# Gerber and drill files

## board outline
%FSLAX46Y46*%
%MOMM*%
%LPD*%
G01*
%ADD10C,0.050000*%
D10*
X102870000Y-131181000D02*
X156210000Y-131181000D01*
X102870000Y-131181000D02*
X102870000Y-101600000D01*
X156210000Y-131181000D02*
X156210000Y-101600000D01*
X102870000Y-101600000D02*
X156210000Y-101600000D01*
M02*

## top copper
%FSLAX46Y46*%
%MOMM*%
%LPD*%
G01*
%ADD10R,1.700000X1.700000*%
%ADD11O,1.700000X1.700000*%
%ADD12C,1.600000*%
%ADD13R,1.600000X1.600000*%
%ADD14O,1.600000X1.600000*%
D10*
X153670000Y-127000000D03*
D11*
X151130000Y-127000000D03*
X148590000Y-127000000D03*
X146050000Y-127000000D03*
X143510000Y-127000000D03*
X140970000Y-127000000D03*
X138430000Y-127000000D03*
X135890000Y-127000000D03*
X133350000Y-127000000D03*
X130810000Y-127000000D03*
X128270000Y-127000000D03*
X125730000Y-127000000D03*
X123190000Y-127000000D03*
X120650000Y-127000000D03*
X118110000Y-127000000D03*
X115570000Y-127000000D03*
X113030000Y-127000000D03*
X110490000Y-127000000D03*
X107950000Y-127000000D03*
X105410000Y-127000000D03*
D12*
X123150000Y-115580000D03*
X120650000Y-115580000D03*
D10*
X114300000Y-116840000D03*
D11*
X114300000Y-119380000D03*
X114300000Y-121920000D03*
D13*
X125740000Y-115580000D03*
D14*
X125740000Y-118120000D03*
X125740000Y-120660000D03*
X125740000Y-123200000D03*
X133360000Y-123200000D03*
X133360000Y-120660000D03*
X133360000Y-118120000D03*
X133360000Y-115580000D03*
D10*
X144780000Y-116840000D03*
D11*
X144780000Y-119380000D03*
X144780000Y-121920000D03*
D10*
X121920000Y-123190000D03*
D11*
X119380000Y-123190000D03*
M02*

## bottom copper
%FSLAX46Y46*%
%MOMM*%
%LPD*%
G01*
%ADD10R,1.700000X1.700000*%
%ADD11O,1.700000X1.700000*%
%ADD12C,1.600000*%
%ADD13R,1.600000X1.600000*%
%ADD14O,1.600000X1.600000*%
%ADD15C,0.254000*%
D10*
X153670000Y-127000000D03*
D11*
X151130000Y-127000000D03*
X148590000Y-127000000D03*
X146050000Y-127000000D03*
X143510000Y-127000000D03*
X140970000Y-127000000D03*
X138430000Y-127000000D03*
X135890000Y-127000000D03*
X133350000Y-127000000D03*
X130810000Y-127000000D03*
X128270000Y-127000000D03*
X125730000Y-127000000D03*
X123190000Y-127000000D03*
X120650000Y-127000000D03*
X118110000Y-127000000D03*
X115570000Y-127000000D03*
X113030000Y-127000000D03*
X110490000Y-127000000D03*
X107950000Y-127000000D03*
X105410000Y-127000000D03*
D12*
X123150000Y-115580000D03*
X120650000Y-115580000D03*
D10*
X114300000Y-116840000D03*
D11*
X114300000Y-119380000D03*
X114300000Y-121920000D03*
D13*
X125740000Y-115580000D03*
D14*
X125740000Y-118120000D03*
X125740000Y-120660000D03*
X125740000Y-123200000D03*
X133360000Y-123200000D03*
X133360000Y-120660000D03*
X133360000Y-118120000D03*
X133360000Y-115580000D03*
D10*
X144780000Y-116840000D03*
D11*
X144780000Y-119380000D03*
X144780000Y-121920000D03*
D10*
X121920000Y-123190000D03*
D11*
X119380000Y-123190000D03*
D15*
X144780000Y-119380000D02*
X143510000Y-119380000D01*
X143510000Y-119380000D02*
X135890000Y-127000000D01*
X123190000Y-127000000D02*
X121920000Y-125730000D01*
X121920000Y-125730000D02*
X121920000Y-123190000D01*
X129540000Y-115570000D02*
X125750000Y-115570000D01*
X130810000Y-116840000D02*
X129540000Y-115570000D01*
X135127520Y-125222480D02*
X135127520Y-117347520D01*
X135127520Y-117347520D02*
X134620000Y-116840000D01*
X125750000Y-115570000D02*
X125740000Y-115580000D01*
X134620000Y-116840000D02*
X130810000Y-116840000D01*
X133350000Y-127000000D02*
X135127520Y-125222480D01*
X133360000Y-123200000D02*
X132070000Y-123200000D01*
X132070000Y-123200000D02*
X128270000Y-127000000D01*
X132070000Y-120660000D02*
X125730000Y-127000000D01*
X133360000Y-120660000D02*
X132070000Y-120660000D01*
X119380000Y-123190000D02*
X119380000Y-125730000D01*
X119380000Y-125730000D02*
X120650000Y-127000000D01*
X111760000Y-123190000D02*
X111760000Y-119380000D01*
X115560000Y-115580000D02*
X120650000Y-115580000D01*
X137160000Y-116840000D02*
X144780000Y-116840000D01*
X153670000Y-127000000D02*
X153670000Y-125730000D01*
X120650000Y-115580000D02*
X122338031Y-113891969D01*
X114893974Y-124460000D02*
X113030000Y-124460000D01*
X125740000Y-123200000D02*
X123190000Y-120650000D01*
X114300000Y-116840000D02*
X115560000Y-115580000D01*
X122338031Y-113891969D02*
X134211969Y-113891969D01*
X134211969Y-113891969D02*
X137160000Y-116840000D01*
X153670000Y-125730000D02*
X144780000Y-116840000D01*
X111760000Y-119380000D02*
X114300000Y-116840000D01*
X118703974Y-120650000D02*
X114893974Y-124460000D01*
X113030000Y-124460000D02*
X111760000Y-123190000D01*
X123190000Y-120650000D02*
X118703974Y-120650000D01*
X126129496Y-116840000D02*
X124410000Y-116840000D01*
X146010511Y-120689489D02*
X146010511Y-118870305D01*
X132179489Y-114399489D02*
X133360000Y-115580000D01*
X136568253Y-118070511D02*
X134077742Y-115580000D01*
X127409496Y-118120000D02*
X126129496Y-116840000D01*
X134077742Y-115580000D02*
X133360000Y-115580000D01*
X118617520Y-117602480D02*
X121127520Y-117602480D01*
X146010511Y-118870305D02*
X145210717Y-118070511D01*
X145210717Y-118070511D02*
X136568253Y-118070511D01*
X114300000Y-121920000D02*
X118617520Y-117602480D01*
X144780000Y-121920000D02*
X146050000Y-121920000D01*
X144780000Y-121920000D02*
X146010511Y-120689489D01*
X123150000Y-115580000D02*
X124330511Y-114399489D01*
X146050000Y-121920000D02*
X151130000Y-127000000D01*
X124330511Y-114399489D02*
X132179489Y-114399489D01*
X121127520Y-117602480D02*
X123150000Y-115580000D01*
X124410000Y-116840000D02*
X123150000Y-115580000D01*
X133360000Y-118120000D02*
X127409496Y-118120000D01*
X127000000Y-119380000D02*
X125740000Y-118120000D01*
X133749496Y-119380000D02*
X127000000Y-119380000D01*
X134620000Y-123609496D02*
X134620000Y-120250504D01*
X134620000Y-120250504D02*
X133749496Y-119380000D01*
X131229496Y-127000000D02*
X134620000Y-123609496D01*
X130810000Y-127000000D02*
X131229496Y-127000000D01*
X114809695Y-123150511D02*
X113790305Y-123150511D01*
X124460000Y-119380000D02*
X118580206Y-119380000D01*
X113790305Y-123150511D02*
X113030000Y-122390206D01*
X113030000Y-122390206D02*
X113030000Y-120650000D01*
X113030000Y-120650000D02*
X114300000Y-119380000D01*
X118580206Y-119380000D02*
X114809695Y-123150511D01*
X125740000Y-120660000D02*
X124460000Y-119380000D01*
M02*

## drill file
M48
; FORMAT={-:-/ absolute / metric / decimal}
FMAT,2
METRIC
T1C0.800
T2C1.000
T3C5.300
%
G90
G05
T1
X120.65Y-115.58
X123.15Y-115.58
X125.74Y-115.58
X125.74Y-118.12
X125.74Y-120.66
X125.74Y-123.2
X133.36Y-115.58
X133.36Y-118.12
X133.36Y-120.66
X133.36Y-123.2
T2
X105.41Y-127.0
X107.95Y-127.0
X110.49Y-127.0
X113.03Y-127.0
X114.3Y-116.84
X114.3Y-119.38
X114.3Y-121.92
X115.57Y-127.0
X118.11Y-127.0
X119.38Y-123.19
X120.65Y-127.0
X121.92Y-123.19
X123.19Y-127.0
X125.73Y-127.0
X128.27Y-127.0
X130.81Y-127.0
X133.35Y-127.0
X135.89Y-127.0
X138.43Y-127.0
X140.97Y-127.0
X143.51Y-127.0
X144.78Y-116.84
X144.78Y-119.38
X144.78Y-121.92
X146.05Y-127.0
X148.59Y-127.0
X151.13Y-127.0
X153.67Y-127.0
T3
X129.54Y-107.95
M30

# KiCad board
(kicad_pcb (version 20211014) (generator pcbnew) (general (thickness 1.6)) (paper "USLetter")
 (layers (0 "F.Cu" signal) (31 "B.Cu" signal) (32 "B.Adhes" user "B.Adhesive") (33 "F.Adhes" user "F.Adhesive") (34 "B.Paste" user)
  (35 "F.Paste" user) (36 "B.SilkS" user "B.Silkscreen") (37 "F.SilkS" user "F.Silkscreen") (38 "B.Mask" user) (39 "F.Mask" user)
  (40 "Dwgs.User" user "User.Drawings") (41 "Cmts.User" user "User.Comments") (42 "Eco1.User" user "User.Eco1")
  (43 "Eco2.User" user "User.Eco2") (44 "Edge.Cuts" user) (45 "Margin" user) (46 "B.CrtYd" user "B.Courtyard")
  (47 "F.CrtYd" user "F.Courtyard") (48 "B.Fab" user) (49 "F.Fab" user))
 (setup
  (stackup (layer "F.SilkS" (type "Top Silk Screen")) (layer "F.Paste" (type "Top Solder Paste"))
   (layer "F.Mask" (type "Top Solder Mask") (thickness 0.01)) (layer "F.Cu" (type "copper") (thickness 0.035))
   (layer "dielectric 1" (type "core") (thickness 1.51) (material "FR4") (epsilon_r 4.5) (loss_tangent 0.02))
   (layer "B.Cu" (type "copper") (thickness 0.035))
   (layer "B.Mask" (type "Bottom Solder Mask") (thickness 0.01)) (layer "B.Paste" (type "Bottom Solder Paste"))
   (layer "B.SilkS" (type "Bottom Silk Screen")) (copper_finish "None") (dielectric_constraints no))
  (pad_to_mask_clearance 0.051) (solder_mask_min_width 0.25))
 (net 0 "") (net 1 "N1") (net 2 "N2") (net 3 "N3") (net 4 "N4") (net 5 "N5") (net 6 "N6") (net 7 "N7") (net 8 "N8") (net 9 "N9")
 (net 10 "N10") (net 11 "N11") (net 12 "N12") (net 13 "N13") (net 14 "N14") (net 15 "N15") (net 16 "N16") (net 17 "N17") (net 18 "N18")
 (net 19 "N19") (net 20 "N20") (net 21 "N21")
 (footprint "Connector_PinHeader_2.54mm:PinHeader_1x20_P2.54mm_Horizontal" (layer "F.Cu") (at 153.67 127 -90)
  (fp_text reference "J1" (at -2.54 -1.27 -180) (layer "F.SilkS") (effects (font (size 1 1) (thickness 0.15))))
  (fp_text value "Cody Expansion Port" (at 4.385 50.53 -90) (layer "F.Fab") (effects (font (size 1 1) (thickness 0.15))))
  (pad "1" thru_hole rect (at 0 0 270) (size 1.7 1.7) (drill 1) (layers *.Cu *.Mask) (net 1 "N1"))
  (pad "2" thru_hole oval (at 0 2.54 270) (size 1.7 1.7) (drill 1) (layers *.Cu *.Mask) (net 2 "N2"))
  (pad "3" thru_hole oval (at 0 5.08 270) (size 1.7 1.7) (drill 1) (layers *.Cu *.Mask) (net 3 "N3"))
  (pad "4" thru_hole oval (at 0 7.62 270) (size 1.7 1.7) (drill 1) (layers *.Cu *.Mask) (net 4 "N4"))
  (pad "5" thru_hole oval (at 0 10.16 270) (size 1.7 1.7) (drill 1) (layers *.Cu *.Mask) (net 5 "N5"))
  (pad "6" thru_hole oval (at 0 12.7 270) (size 1.7 1.7) (drill 1) (layers *.Cu *.Mask) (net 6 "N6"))
  (pad "7" thru_hole oval (at 0 15.24 270) (size 1.7 1.7) (drill 1) (layers *.Cu *.Mask) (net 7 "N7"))
  (pad "8" thru_hole oval (at 0 17.78 270) (size 1.7 1.7) (drill 1) (layers *.Cu *.Mask) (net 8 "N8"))
  (pad "9" thru_hole oval (at 0 20.32 270) (size 1.7 1.7) (drill 1) (layers *.Cu *.Mask) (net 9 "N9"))
  (pad "10" thru_hole oval (at 0 22.86 270) (size 1.7 1.7) (drill 1) (layers *.Cu *.Mask) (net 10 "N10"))
  (pad "11" thru_hole oval (at 0 25.4 270) (size 1.7 1.7) (drill 1) (layers *.Cu *.Mask) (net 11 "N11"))
  (pad "12" thru_hole oval (at 0 27.94 270) (size 1.7 1.7) (drill 1) (layers *.Cu *.Mask) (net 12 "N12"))
  (pad "13" thru_hole oval (at 0 30.48 270) (size 1.7 1.7) (drill 1) (layers *.Cu *.Mask) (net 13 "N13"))
  (pad "14" thru_hole oval (at 0 33.02 270) (size 1.7 1.7) (drill 1) (layers *.Cu *.Mask) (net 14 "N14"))
  (pad "15" thru_hole oval (at 0 35.56 270) (size 1.7 1.7) (drill 1) (layers *.Cu *.Mask) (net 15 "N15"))
  (pad "16" thru_hole oval (at 0 38.1 270) (size 1.7 1.7) (drill 1) (layers *.Cu *.Mask) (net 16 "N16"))
  (pad "17" thru_hole oval (at 0 40.64 270) (size 1.7 1.7) (drill 1) (layers *.Cu *.Mask) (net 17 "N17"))
  (pad "18" thru_hole oval (at 0 43.18 270) (size 1.7 1.7) (drill 1) (layers *.Cu *.Mask) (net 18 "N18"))
  (pad "19" thru_hole oval (at 0 45.72 270) (size 1.7 1.7) (drill 1) (layers *.Cu *.Mask) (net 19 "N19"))
  (pad "20" thru_hole oval (at 0 48.26 270) (size 1.7 1.7) (drill 1) (layers *.Cu *.Mask) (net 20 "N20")))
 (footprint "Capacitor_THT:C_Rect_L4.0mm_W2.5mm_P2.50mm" (layer "F.Cu") (at 123.15 115.58 180)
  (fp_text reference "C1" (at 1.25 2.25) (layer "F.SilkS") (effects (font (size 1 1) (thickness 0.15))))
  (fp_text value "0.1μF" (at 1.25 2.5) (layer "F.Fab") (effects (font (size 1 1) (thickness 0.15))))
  (pad "1" thru_hole circle (at 0 0 180) (size 1.6 1.6) (drill 0.8) (layers *.Cu *.Mask) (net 2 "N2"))
  (pad "2" thru_hole circle (at 2.5 0 180) (size 1.6 1.6) (drill 0.8) (layers *.Cu *.Mask) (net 1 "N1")))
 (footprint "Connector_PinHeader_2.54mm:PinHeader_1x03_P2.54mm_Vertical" (layer "F.Cu") (at 114.3 116.84)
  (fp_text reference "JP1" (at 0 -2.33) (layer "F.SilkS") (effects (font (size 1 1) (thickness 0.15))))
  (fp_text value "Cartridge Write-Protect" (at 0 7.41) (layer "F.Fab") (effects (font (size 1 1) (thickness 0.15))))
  (pad "1" thru_hole rect (at 0 0) (size 1.7 1.7) (drill 1) (layers *.Cu *.Mask) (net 1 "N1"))
  (pad "2" thru_hole oval (at 0 2.54) (size 1.7 1.7) (drill 1) (layers *.Cu *.Mask) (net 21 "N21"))
  (pad "3" thru_hole oval (at 0 5.08) (size 1.7 1.7) (drill 1) (layers *.Cu *.Mask) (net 2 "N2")))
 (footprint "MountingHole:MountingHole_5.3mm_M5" (layer "F.Cu") (at 129.54 107.95)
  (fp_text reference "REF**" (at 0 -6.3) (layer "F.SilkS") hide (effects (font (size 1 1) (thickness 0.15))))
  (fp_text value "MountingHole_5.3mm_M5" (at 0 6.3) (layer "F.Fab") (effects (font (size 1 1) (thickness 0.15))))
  (pad "" np_thru_hole circle (at 0 0) (size 5.3 5.3) (drill 5.3) (layers *.Cu *.Mask)))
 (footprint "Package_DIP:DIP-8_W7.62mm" (layer "F.Cu") (at 125.74 115.58)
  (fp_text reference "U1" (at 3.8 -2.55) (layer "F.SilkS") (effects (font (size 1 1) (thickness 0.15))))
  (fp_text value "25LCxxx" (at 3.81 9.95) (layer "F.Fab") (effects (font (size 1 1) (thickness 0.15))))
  (pad "1" thru_hole rect (at 0 0) (size 1.6 1.6) (drill 0.8) (layers *.Cu *.Mask) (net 9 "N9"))
  (pad "2" thru_hole oval (at 0 2.54) (size 1.6 1.6) (drill 0.8) (layers *.Cu *.Mask) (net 10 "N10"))
  (pad "3" thru_hole oval (at 0 5.08) (size 1.6 1.6) (drill 0.8) (layers *.Cu *.Mask) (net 21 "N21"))
  (pad "4" thru_hole oval (at 0 7.62) (size 1.6 1.6) (drill 0.8) (layers *.Cu *.Mask) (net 1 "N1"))
  (pad "5" thru_hole oval (at 7.62 7.62) (size 1.6 1.6) (drill 0.8) (layers *.Cu *.Mask) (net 11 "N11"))
  (pad "6" thru_hole oval (at 7.62 5.08) (size 1.6 1.6) (drill 0.8) (layers *.Cu *.Mask) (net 12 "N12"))
  (pad "7" thru_hole oval (at 7.62 2.54) (size 1.6 1.6) (drill 0.8) (layers *.Cu *.Mask) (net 2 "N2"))
  (pad "8" thru_hole oval (at 7.62 0) (size 1.6 1.6) (drill 0.8) (layers *.Cu *.Mask) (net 2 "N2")))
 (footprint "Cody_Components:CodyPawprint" (layer "F.Cu") (at 109.22 106.68)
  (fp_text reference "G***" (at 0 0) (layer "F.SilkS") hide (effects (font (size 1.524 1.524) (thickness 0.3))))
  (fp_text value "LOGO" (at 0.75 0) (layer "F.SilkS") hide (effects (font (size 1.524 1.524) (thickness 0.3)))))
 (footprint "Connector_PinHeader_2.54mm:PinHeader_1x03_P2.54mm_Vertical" (layer "F.Cu") (at 144.78 116.84)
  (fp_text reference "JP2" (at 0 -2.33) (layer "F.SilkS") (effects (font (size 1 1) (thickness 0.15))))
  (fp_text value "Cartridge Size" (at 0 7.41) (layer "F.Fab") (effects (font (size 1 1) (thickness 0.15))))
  (pad "1" thru_hole rect (at 0 0) (size 1.7 1.7) (drill 1) (layers *.Cu *.Mask) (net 1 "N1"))
  (pad "2" thru_hole oval (at 0 2.54) (size 1.7 1.7) (drill 1) (layers *.Cu *.Mask) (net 8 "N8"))
  (pad "3" thru_hole oval (at 0 5.08) (size 1.7 1.7) (drill 1) (layers *.Cu *.Mask) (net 2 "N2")))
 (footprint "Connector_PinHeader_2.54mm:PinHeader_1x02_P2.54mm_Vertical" (layer "F.Cu") (at 121.92 123.19 -90)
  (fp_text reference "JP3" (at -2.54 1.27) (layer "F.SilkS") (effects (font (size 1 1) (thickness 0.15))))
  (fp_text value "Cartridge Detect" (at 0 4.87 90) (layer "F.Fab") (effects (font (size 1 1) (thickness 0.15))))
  (pad "1" thru_hole rect (at 0 0 270) (size 1.7 1.7) (drill 1) (layers *.Cu *.Mask) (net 13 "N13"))
  (pad "2" thru_hole oval (at 0 2.54 270) (size 1.7 1.7) (drill 1) (layers *.Cu *.Mask) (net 14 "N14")))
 (gr_line (start 102.87 131.181) (end 156.21 131.181) (layer "Edge.Cuts") (width 0.05))
 (gr_line (start 102.87 131.181) (end 102.87 101.6) (layer "Edge.Cuts") (width 0.05))
 (gr_line (start 156.21 131.181) (end 156.21 101.6) (layer "Edge.Cuts") (width 0.05))
 (gr_line (start 102.87 101.6) (end 156.21 101.6) (layer "Edge.Cuts") (width 0.05))
 (segment (start 144.78 119.38) (end 143.51 119.38) (width 0.254) (layer "B.Cu") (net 8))
 (segment (start 143.51 119.38) (end 135.89 127) (width 0.254) (layer "B.Cu") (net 8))
 (segment (start 123.19 127) (end 121.92 125.73) (width 0.254) (layer "B.Cu") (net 13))
 (segment (start 121.92 125.73) (end 121.92 123.19) (width 0.254) (layer "B.Cu") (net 13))
 (segment (start 129.54 115.57) (end 125.75 115.57) (width 0.254) (layer "B.Cu") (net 9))
 (segment (start 130.81 116.84) (end 129.54 115.57) (width 0.254) (layer "B.Cu") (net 9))
 (segment (start 135.12752 125.22248) (end 135.12752 117.34752) (width 0.254) (layer "B.Cu") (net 9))
 (segment (start 135.12752 117.34752) (end 134.62 116.84) (width 0.254) (layer "B.Cu") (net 9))
 (segment (start 125.75 115.57) (end 125.74 115.58) (width 0.254) (layer "B.Cu") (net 9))
 (segment (start 134.62 116.84) (end 130.81 116.84) (width 0.254) (layer "B.Cu") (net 9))
 (segment (start 133.35 127) (end 135.12752 125.22248) (width 0.254) (layer "B.Cu") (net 9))
 (segment (start 133.36 123.2) (end 132.07 123.2) (width 0.254) (layer "B.Cu") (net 11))
 (segment (start 132.07 123.2) (end 128.27 127) (width 0.254) (layer "B.Cu") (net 11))
 (segment (start 132.07 120.66) (end 125.73 127) (width 0.254) (layer "B.Cu") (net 12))
 (segment (start 133.36 120.66) (end 132.07 120.66) (width 0.254) (layer "B.Cu") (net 12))
 (segment (start 119.38 123.19) (end 119.38 125.73) (width 0.254) (layer "B.Cu") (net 14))
 (segment (start 119.38 125.73) (end 120.65 127) (width 0.254) (layer "B.Cu") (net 14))
 (segment (start 111.76 123.19) (end 111.76 119.38) (width 0.254) (layer "B.Cu") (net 1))
 (segment (start 115.56 115.58) (end 120.65 115.58) (width 0.254) (layer "B.Cu") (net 1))
 (segment (start 137.16 116.84) (end 144.78 116.84) (width 0.254) (layer "B.Cu") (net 1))
 (segment (start 153.67 127) (end 153.67 125.73) (width 0.254) (layer "B.Cu") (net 1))
 (segment (start 120.65 115.58) (end 122.338031 113.891969) (width 0.254) (layer "B.Cu") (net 1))
 (segment (start 114.893974 124.46) (end 113.03 124.46) (width 0.254) (layer "B.Cu") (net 1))
 (segment (start 125.74 123.2) (end 123.19 120.65) (width 0.254) (layer "B.Cu") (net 1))
 (segment (start 114.3 116.84) (end 115.56 115.58) (width 0.254) (layer "B.Cu") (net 1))
 (segment (start 122.338031 113.891969) (end 134.211969 113.891969) (width 0.254) (layer "B.Cu") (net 1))
 (segment (start 134.211969 113.891969) (end 137.16 116.84) (width 0.254) (layer "B.Cu") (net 1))
 (segment (start 153.67 125.73) (end 144.78 116.84) (width 0.254) (layer "B.Cu") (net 1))
 (segment (start 111.76 119.38) (end 114.3 116.84) (width 0.254) (layer "B.Cu") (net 1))
 (segment (start 118.703974 120.65) (end 114.893974 124.46) (width 0.254) (layer "B.Cu") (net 1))
 (segment (start 113.03 124.46) (end 111.76 123.19) (width 0.254) (layer "B.Cu") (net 1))
 (segment (start 123.19 120.65) (end 118.703974 120.65) (width 0.254) (layer "B.Cu") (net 1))
 (segment (start 126.129496 116.84) (end 124.41 116.84) (width 0.254) (layer "B.Cu") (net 2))
 (segment (start 146.010511 120.689489) (end 146.010511 118.870305) (width 0.254) (layer "B.Cu") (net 2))
 (segment (start 132.179489 114.399489) (end 133.36 115.58) (width 0.254) (layer "B.Cu") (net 2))
 (segment (start 136.568253 118.070511) (end 134.077742 115.58) (width 0.254) (layer "B.Cu") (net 2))
 (segment (start 127.409496 118.12) (end 126.129496 116.84) (width 0.254) (layer "B.Cu") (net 2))
 (segment (start 134.077742 115.58) (end 133.36 115.58) (width 0.254) (layer "B.Cu") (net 2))
 (segment (start 118.61752 117.60248) (end 121.12752 117.60248) (width 0.254) (layer "B.Cu") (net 2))
 (segment (start 146.010511 118.870305) (end 145.210717 118.070511) (width 0.254) (layer "B.Cu") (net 2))
 (segment (start 145.210717 118.070511) (end 136.568253 118.070511) (width 0.254) (layer "B.Cu") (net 2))
 (segment (start 114.3 121.92) (end 118.61752 117.60248) (width 0.254) (layer "B.Cu") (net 2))
 (segment (start 144.78 121.92) (end 146.05 121.92) (width 0.254) (layer "B.Cu") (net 2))
 (segment (start 144.78 121.92) (end 146.010511 120.689489) (width 0.254) (layer "B.Cu") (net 2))
 (segment (start 123.15 115.58) (end 124.330511 114.399489) (width 0.254) (layer "B.Cu") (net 2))
 (segment (start 146.05 121.92) (end 151.13 127) (width 0.254) (layer "B.Cu") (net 2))
 (segment (start 124.330511 114.399489) (end 132.179489 114.399489) (width 0.254) (layer "B.Cu") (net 2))
 (segment (start 121.12752 117.60248) (end 123.15 115.58) (width 0.254) (layer "B.Cu") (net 2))
 (segment (start 124.41 116.84) (end 123.15 115.58) (width 0.254) (layer "B.Cu") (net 2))
 (segment (start 133.36 118.12) (end 127.409496 118.12) (width 0.254) (layer "B.Cu") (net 2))
 (segment (start 127 119.38) (end 125.74 118.12) (width 0.254) (layer "B.Cu") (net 10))
 (segment (start 133.749496 119.38) (end 127 119.38) (width 0.254) (layer "B.Cu") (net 10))
 (segment (start 134.62 123.609496) (end 134.62 120.250504) (width 0.254) (layer "B.Cu") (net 10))
 (segment (start 134.62 120.250504) (end 133.749496 119.38) (width 0.254) (layer "B.Cu") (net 10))
 (segment (start 131.229496 127) (end 134.62 123.609496) (width 0.254) (layer "B.Cu") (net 10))
 (segment (start 130.81 127) (end 131.229496 127) (width 0.254) (layer "B.Cu") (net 10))
 (segment (start 114.809695 123.150511) (end 113.790305 123.150511) (width 0.254) (layer "B.Cu") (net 21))
 (segment (start 124.46 119.38) (end 118.580206 119.38) (width 0.254) (layer "B.Cu") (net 21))
 (segment (start 113.790305 123.150511) (end 113.03 122.390206) (width 0.254) (layer "B.Cu") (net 21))
 (segment (start 113.03 122.390206) (end 113.03 120.65) (width 0.254) (layer "B.Cu") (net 21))
 (segment (start 113.03 120.65) (end 114.3 119.38) (width 0.254) (layer "B.Cu") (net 21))
 (segment (start 118.580206 119.38) (end 114.809695 123.150511) (width 0.254) (layer "B.Cu") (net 21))
 (segment (start 125.74 120.66) (end 124.46 119.38) (width 0.254) (layer "B.Cu") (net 21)))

